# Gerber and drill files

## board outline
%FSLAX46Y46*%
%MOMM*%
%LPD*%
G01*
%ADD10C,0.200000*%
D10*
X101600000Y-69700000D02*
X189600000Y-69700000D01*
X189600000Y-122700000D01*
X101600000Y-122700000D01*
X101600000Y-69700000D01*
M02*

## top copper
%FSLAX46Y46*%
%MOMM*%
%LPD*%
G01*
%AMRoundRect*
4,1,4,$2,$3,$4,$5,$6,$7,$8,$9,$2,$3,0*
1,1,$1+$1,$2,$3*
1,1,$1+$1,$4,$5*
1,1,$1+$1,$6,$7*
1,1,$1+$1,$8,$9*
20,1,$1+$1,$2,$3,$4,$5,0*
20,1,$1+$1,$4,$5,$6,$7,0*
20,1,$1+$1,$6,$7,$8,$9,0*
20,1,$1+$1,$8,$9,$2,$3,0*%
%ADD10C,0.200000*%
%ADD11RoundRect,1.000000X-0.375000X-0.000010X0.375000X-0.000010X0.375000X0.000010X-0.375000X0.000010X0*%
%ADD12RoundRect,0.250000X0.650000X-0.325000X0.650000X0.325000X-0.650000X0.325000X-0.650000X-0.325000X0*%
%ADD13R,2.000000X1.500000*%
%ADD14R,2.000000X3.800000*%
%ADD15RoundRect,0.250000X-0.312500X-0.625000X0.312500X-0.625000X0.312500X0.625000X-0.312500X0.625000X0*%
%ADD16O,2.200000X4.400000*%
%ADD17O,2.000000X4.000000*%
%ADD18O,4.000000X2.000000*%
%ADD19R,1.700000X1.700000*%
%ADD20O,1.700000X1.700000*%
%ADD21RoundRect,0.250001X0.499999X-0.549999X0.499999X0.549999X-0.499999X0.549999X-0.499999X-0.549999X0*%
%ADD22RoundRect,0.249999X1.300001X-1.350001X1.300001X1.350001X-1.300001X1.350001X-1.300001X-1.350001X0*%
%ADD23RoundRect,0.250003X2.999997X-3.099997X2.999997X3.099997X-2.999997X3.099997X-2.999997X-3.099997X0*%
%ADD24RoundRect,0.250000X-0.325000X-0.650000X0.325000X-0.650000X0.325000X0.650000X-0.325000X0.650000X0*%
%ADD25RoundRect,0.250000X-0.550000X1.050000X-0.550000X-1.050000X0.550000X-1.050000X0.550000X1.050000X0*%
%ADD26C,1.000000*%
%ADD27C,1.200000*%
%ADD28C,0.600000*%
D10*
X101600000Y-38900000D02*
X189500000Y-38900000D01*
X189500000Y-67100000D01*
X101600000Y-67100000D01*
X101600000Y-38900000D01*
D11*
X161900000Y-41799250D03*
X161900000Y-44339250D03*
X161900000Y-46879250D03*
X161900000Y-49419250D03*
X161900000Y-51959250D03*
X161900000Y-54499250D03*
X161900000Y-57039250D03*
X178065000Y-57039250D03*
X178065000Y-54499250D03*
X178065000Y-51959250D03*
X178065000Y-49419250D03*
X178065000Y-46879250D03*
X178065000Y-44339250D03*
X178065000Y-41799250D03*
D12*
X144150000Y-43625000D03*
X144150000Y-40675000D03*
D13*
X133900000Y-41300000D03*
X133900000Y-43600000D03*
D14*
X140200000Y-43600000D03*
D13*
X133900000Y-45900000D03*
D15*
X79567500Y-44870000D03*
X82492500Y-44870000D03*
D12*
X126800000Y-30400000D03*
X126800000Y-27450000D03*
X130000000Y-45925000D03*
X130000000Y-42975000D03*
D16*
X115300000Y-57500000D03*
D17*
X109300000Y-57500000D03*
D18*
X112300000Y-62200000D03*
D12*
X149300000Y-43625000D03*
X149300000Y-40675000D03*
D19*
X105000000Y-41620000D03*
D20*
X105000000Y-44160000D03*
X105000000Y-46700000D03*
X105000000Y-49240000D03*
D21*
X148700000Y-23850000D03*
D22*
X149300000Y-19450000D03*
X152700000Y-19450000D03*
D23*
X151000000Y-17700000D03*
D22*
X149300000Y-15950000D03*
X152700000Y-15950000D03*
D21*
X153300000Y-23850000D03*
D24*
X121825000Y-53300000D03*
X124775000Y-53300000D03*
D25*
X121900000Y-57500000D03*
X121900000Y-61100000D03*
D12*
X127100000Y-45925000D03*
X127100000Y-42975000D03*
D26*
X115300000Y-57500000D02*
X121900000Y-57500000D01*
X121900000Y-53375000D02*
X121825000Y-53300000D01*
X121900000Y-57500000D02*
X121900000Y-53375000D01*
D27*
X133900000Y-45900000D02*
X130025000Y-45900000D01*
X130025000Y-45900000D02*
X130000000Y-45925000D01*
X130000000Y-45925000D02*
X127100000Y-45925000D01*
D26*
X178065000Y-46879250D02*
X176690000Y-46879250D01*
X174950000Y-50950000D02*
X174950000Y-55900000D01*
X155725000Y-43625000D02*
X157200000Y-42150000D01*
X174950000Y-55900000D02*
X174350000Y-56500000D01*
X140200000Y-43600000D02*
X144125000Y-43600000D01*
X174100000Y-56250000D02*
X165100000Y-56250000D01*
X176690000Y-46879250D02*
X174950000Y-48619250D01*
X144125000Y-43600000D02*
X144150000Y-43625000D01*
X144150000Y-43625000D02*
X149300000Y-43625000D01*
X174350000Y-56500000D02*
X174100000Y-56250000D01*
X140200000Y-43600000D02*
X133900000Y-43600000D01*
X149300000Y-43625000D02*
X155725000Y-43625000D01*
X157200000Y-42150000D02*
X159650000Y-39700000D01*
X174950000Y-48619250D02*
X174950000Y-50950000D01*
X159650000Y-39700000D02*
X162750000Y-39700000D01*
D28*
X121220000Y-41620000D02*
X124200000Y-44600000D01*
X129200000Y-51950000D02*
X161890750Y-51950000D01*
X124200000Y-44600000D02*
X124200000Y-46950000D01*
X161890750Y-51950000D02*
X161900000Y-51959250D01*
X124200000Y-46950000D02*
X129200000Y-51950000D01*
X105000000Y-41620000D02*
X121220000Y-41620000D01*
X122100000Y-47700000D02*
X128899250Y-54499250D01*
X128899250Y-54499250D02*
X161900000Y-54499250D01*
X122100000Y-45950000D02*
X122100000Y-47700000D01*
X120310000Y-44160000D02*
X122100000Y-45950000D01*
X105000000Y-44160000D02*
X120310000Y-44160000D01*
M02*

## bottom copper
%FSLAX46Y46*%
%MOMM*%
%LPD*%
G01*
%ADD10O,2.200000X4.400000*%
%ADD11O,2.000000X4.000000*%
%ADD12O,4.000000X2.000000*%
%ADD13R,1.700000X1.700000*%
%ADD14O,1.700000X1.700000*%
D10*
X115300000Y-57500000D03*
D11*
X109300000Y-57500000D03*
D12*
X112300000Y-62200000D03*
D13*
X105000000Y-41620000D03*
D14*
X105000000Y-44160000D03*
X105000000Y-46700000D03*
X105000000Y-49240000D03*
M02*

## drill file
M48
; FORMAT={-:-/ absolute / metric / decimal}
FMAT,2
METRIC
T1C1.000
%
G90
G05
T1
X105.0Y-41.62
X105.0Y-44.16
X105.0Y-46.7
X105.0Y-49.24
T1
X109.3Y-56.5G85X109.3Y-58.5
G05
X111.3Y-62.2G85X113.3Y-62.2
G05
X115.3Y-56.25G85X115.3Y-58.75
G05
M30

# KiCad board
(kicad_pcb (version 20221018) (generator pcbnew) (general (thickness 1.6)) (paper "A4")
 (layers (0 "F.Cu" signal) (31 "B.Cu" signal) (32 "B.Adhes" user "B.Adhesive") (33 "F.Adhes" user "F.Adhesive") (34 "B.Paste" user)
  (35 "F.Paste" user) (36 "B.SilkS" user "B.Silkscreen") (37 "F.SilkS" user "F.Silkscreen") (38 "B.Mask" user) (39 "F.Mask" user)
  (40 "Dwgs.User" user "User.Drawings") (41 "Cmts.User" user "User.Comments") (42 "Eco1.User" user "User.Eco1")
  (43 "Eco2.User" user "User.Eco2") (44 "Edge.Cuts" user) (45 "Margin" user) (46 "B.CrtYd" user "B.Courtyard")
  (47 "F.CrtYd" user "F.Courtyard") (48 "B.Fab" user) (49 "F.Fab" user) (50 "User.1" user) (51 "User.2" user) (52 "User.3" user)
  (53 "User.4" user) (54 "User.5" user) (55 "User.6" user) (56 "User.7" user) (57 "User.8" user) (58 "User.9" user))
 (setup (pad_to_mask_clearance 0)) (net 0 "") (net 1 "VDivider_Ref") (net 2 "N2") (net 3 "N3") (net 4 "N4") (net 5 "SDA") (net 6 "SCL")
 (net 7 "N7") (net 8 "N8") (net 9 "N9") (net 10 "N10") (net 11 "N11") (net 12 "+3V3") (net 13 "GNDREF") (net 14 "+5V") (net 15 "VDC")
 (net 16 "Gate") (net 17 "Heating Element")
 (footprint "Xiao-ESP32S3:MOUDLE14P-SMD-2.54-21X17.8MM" (layer "F.Cu") (at 161.065 59.91925)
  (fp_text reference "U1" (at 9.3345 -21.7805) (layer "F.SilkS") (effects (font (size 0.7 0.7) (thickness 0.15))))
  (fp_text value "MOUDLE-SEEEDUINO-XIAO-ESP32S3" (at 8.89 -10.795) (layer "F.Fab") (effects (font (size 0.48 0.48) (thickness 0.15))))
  (pad "1" smd roundrect (at 0.835 -18.12) (size 2.75 2) (layers "F.Cu" "F.Paste" "F.Mask") (roundrect_rratio 0.5) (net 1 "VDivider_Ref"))
  (pad "2" smd roundrect (at 0.835 -15.58) (size 2.75 2) (layers "F.Cu" "F.Paste" "F.Mask") (roundrect_rratio 0.5) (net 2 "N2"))
  (pad "3" smd roundrect (at 0.835 -13.04) (size 2.75 2) (layers "F.Cu" "F.Paste" "F.Mask") (roundrect_rratio 0.5) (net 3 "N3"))
  (pad "4" smd roundrect (at 0.835 -10.5) (size 2.75 2) (layers "F.Cu" "F.Paste" "F.Mask") (roundrect_rratio 0.5) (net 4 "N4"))
  (pad "5" smd roundrect (at 0.835 -7.96) (size 2.75 2) (layers "F.Cu" "F.Paste" "F.Mask") (roundrect_rratio 0.5) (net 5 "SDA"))
  (pad "6" smd roundrect (at 0.835 -5.42) (size 2.75 2) (layers "F.Cu" "F.Paste" "F.Mask") (roundrect_rratio 0.5) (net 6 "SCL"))
  (pad "7" smd roundrect (at 0.835 -2.88) (size 2.75 2) (layers "F.Cu" "F.Paste" "F.Mask") (roundrect_rratio 0.5) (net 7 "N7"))
  (pad "8" smd roundrect (at 17 -2.88) (size 2.75 2) (layers "F.Cu" "F.Paste" "F.Mask") (roundrect_rratio 0.5) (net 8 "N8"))
  (pad "9" smd roundrect (at 17 -5.42) (size 2.75 2) (layers "F.Cu" "F.Paste" "F.Mask") (roundrect_rratio 0.5) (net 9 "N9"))
  (pad "10" smd roundrect (at 17 -7.96) (size 2.75 2) (layers "F.Cu" "F.Paste" "F.Mask") (roundrect_rratio 0.5) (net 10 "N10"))
  (pad "11" smd roundrect (at 17 -10.5) (size 2.75 2) (layers "F.Cu" "F.Paste" "F.Mask") (roundrect_rratio 0.5) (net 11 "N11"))
  (pad "12" smd roundrect (at 17 -13.04) (size 2.75 2) (layers "F.Cu" "F.Paste" "F.Mask") (roundrect_rratio 0.5) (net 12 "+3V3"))
  (pad "13" smd roundrect (at 17 -15.58) (size 2.75 2) (layers "F.Cu" "F.Paste" "F.Mask") (roundrect_rratio 0.5) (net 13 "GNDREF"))
  (pad "14" smd roundrect (at 17 -18.12) (size 2.75 2) (layers "F.Cu" "F.Paste" "F.Mask") (roundrect_rratio 0.5) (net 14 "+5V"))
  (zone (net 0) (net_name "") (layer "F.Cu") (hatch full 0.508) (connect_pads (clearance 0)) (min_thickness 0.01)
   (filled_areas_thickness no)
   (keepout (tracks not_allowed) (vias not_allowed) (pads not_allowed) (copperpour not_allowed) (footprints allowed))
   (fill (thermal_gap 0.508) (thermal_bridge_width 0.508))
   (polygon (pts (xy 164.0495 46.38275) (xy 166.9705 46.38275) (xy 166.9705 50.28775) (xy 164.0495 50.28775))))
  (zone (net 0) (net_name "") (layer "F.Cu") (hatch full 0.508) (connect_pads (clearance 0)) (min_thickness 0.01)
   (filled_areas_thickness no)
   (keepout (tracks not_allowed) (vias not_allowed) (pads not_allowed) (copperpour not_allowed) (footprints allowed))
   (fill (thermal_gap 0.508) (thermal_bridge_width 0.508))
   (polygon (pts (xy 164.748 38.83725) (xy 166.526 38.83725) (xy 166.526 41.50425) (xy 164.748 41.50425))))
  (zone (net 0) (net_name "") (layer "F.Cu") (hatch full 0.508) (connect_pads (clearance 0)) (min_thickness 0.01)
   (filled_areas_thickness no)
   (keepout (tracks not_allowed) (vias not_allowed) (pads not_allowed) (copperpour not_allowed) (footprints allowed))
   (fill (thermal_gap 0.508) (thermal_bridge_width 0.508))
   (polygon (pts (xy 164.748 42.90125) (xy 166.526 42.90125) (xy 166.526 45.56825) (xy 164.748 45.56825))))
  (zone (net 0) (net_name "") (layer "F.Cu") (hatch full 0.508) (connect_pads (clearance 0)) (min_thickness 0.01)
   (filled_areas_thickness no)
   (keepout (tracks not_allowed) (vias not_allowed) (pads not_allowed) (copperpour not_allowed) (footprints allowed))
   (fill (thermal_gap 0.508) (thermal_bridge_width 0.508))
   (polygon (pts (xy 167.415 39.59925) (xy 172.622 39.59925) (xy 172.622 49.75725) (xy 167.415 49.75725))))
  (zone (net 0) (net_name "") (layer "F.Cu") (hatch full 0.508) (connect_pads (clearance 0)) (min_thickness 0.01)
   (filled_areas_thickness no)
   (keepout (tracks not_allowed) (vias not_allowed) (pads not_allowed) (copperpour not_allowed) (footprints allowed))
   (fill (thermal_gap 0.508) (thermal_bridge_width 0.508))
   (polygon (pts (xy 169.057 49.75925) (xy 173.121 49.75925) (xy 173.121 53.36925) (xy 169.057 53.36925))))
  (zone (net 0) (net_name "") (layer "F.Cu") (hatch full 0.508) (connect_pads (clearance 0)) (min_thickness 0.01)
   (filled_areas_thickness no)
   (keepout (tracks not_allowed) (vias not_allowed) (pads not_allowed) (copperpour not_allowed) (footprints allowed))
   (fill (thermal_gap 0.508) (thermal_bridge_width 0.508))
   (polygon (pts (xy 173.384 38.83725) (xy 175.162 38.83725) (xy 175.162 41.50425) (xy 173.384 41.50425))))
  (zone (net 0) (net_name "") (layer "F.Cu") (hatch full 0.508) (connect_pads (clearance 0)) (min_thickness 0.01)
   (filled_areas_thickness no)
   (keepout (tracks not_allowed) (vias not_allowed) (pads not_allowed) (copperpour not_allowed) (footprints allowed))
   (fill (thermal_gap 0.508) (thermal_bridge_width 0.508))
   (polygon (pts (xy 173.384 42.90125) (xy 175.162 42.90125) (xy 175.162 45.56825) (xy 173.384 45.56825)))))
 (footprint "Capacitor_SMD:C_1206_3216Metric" (layer "F.Cu") (at 144.15 42.15 90)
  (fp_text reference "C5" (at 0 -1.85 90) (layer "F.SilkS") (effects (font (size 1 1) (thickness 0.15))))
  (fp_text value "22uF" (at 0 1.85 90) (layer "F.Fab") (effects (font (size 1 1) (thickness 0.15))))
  (pad "1" smd roundrect (at -1.475 0 90) (size 1.15 1.8) (layers "F.Cu" "F.Paste" "F.Mask") (roundrect_rratio 0.217391) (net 12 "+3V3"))
  (pad "2" smd roundrect (at 1.475 0 90) (size 1.15 1.8) (layers "F.Cu" "F.Paste" "F.Mask") (roundrect_rratio 0.217391) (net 13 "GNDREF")))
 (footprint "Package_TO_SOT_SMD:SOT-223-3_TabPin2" (layer "F.Cu") (at 137.05 43.6)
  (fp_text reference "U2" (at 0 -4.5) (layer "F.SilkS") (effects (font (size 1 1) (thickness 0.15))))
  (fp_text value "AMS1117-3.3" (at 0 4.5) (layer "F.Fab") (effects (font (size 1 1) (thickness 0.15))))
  (pad "1" smd rect (at -3.15 -2.3) (size 2 1.5) (layers "F.Cu" "F.Paste" "F.Mask") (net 13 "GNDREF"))
  (pad "2" smd rect (at -3.15 0) (size 2 1.5) (layers "F.Cu" "F.Paste" "F.Mask") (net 12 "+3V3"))
  (pad "2" smd rect (at 3.15 0) (size 2 3.8) (layers "F.Cu" "F.Paste" "F.Mask") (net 12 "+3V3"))
  (pad "3" smd rect (at -3.15 2.3) (size 2 1.5) (layers "F.Cu" "F.Paste" "F.Mask") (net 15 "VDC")))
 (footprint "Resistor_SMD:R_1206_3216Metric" (layer "F.Cu") (at 81.03 44.87)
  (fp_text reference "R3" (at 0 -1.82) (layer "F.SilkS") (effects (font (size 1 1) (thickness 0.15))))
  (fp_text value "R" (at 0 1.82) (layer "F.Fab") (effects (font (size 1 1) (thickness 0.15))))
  (pad "1" smd roundrect (at -1.4625 0) (size 1.125 1.75) (layers "F.Cu" "F.Paste" "F.Mask") (roundrect_rratio 0.222222) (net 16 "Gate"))
  (pad "2" smd roundrect (at 1.4625 0) (size 1.125 1.75) (layers "F.Cu" "F.Paste" "F.Mask") (roundrect_rratio 0.222222) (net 13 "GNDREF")))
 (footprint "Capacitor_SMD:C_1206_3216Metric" (layer "F.Cu") (at 126.8 28.925 90)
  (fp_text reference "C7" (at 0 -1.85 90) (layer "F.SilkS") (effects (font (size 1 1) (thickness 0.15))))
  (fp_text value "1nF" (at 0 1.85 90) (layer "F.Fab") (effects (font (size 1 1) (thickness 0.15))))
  (pad "1" smd roundrect (at -1.475 0 90) (size 1.15 1.8) (layers "F.Cu" "F.Paste" "F.Mask") (roundrect_rratio 0.217391)
   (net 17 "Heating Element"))
  (pad "2" smd roundrect (at 1.475 0 90) (size 1.15 1.8) (layers "F.Cu" "F.Paste" "F.Mask") (roundrect_rratio 0.217391)
   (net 17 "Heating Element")))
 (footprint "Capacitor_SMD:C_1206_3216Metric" (layer "F.Cu") (at 130 44.45 90)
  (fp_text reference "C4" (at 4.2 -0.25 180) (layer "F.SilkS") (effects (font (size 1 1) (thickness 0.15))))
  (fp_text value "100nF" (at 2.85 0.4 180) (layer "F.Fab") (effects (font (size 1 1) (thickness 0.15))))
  (pad "1" smd roundrect (at -1.475 0 90) (size 1.15 1.8) (layers "F.Cu" "F.Paste" "F.Mask") (roundrect_rratio 0.217391) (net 15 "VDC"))
  (pad "2" smd roundrect (at 1.475 0 90) (size 1.15 1.8) (layers "F.Cu" "F.Paste" "F.Mask") (roundrect_rratio 0.217391) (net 13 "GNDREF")))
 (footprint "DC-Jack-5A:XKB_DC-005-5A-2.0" (layer "F.Cu") (at 109.3 57.5)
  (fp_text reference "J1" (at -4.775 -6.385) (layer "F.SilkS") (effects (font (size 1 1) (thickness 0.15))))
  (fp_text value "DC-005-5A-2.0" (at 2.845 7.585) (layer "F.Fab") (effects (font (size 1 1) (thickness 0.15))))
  (pad "1" thru_hole oval (at 6 0) (size 2.2 4.4) (drill oval 1 3.5) (layers "*.Cu" "*.Mask") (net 17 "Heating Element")
   (solder_mask_margin 0.102))
  (pad "2" thru_hole oval (at 0 0) (size 2 4) (drill oval 1 3) (layers "*.Cu" "*.Mask") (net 13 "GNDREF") (solder_mask_margin 0.102))
  (pad "3" thru_hole oval (at 3 4.7) (size 4 2) (drill oval 3 1) (layers "*.Cu" "*.Mask") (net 13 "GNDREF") (solder_mask_margin 0.102)))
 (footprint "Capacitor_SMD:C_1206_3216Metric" (layer "F.Cu") (at 149.3 42.15 90)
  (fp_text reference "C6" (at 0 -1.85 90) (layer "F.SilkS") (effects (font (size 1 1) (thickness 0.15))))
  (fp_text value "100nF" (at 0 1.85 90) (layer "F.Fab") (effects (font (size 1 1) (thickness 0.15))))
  (pad "1" smd roundrect (at -1.475 0 90) (size 1.15 1.8) (layers "F.Cu" "F.Paste" "F.Mask") (roundrect_rratio 0.217391) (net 12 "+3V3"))
  (pad "2" smd roundrect (at 1.475 0 90) (size 1.15 1.8) (layers "F.Cu" "F.Paste" "F.Mask") (roundrect_rratio 0.217391) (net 13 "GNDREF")))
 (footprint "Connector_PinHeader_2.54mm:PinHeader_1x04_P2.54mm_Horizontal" (layer "F.Cu") (at 105 41.62)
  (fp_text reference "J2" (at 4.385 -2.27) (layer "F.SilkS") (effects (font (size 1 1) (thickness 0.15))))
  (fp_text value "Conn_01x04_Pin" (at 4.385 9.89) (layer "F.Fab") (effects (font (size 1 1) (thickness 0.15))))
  (pad "1" thru_hole rect (at 0 0) (size 1.7 1.7) (drill 1) (layers "*.Cu" "*.Mask") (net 5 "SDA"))
  (pad "2" thru_hole oval (at 0 2.54) (size 1.7 1.7) (drill 1) (layers "*.Cu" "*.Mask") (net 6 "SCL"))
  (pad "3" thru_hole oval (at 0 5.08) (size 1.7 1.7) (drill 1) (layers "*.Cu" "*.Mask") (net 12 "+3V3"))
  (pad "4" thru_hole oval (at 0 7.62) (size 1.7 1.7) (drill 1) (layers "*.Cu" "*.Mask") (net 13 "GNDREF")))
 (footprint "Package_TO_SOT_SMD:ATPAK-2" (layer "F.Cu") (at 151 18.9 90)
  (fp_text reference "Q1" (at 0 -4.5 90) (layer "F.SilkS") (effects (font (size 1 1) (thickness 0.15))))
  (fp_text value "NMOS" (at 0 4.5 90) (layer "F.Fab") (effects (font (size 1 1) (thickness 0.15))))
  (pad "1" smd roundrect (at -4.95 -2.3 90) (size 1.6 1.5) (layers "F.Cu" "F.Paste" "F.Mask") (roundrect_rratio 0.166667)
   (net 17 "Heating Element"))
  (pad "2" smd roundrect (at -0.55 -1.7 90) (size 3.2 3.1) (layers "F.Cu" "F.Paste") (roundrect_rratio 0.080645) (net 16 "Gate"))
  (pad "2" smd roundrect (at -0.55 1.7 90) (size 3.2 3.1) (layers "F.Cu" "F.Paste") (roundrect_rratio 0.080645) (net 16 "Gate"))
  (pad "2" smd roundrect (at 1.2 0 90) (size 6.7 6.5) (layers "F.Cu" "F.Mask") (roundrect_rratio 0.038462) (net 16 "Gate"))
  (pad "2" smd roundrect (at 2.95 -1.7 90) (size 3.2 3.1) (layers "F.Cu" "F.Paste") (roundrect_rratio 0.080645) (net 16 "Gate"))
  (pad "2" smd roundrect (at 2.95 1.7 90) (size 3.2 3.1) (layers "F.Cu" "F.Paste") (roundrect_rratio 0.080645) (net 16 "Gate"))
  (pad "3" smd roundrect (at -4.95 2.3 90) (size 1.6 1.5) (layers "F.Cu" "F.Paste" "F.Mask") (roundrect_rratio 0.166667) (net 13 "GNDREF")))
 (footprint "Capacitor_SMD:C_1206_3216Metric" (layer "F.Cu") (at 123.3 53.3)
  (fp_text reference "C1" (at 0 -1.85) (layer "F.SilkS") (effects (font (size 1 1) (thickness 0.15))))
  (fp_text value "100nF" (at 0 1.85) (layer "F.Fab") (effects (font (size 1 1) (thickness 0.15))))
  (pad "1" smd roundrect (at -1.475 0) (size 1.15 1.8) (layers "F.Cu" "F.Paste" "F.Mask") (roundrect_rratio 0.217391)
   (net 17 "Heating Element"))
  (pad "2" smd roundrect (at 1.475 0) (size 1.15 1.8) (layers "F.Cu" "F.Paste" "F.Mask") (roundrect_rratio 0.217391) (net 13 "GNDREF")))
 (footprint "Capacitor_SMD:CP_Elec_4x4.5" (layer "F.Cu") (at 121.9 59.3 -90)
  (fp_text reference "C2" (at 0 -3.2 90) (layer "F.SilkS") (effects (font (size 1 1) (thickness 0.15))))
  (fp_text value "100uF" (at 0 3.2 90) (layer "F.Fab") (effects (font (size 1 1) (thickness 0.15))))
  (pad "1" smd roundrect (at -1.8 0 270) (size 2.6 1.6) (layers "F.Cu" "F.Paste" "F.Mask") (roundrect_rratio 0.15625)
   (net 17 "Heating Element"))
  (pad "2" smd roundrect (at 1.8 0 270) (size 2.6 1.6) (layers "F.Cu" "F.Paste" "F.Mask") (roundrect_rratio 0.15625) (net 13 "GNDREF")))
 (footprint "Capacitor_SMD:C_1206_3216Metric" (layer "F.Cu") (at 127.1 44.45 90)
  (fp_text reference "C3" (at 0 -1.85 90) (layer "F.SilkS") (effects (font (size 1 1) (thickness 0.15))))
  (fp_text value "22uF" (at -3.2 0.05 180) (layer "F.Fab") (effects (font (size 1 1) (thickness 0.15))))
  (pad "1" smd roundrect (at -1.475 0 90) (size 1.15 1.8) (layers "F.Cu" "F.Paste" "F.Mask") (roundrect_rratio 0.217391) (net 15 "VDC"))
  (pad "2" smd roundrect (at 1.475 0 90) (size 1.15 1.8) (layers "F.Cu" "F.Paste" "F.Mask") (roundrect_rratio 0.217391) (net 13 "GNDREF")))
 (gr_rect (start 101.6 38.9) (end 189.5 67.1) (stroke (width 0.2) (type default)) (fill none) (layer "F.Cu"))
 (gr_rect (start 101.6 69.7) (end 189.6 122.7) (stroke (width 0.2) (type default)) (fill none) (layer "Edge.Cuts"))
 (segment (start 115.3 57.5) (end 121.9 57.5) (width 1) (layer "F.Cu") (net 17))
 (segment (start 121.9 53.375) (end 121.825 53.3) (width 1) (layer "F.Cu") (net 17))
 (segment (start 121.9 57.5) (end 121.9 53.375) (width 1) (layer "F.Cu") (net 17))
 (segment (start 133.9 45.9) (end 130.025 45.9) (width 1.2) (layer "F.Cu") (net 15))
 (segment (start 130.025 45.9) (end 130 45.925) (width 1.2) (layer "F.Cu") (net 15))
 (segment (start 130 45.925) (end 127.1 45.925) (width 1.2) (layer "F.Cu") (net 15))
 (segment (start 178.065 46.87925) (end 176.69 46.87925) (width 1) (layer "F.Cu") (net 12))
 (segment (start 174.95 50.95) (end 174.95 55.9) (width 1) (layer "F.Cu") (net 12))
 (segment (start 155.725 43.625) (end 157.2 42.15) (width 1) (layer "F.Cu") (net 12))
 (segment (start 174.95 55.9) (end 174.35 56.5) (width 1) (layer "F.Cu") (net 12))
 (segment (start 140.2 43.6) (end 144.125 43.6) (width 1) (layer "F.Cu") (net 12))
 (segment (start 174.1 56.25) (end 165.1 56.25) (width 1) (layer "F.Cu") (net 12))
 (segment (start 176.69 46.87925) (end 174.95 48.61925) (width 1) (layer "F.Cu") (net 12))
 (segment (start 144.125 43.6) (end 144.15 43.625) (width 1) (layer "F.Cu") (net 12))
 (segment (start 144.15 43.625) (end 149.3 43.625) (width 1) (layer "F.Cu") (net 12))
 (segment (start 174.35 56.5) (end 174.1 56.25) (width 1) (layer "F.Cu") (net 12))
 (segment (start 140.2 43.6) (end 133.9 43.6) (width 1) (layer "F.Cu") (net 12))
 (segment (start 149.3 43.625) (end 155.725 43.625) (width 1) (layer "F.Cu") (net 12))
 (segment (start 157.2 42.15) (end 159.65 39.7) (width 1) (layer "F.Cu") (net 12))
 (segment (start 174.95 48.61925) (end 174.95 50.95) (width 1) (layer "F.Cu") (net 12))
 (segment (start 159.65 39.7) (end 162.75 39.7) (width 1) (layer "F.Cu") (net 12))
 (segment (start 121.22 41.62) (end 124.2 44.6) (width 0.6) (layer "F.Cu") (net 5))
 (segment (start 129.2 51.95) (end 161.89075 51.95) (width 0.6) (layer "F.Cu") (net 5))
 (segment (start 124.2 44.6) (end 124.2 46.95) (width 0.6) (layer "F.Cu") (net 5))
 (segment (start 161.89075 51.95) (end 161.9 51.95925) (width 0.6) (layer "F.Cu") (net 5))
 (segment (start 124.2 46.95) (end 129.2 51.95) (width 0.6) (layer "F.Cu") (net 5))
 (segment (start 105 41.62) (end 121.22 41.62) (width 0.6) (layer "F.Cu") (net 5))
 (segment (start 122.1 47.7) (end 128.89925 54.49925) (width 0.6) (layer "F.Cu") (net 6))
 (segment (start 128.89925 54.49925) (end 161.9 54.49925) (width 0.6) (layer "F.Cu") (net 6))
 (segment (start 122.1 45.95) (end 122.1 47.7) (width 0.6) (layer "F.Cu") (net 6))
 (segment (start 120.31 44.16) (end 122.1 45.95) (width 0.6) (layer "F.Cu") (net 6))
 (segment (start 105 44.16) (end 120.31 44.16) (width 0.6) (layer "F.Cu") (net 6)))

